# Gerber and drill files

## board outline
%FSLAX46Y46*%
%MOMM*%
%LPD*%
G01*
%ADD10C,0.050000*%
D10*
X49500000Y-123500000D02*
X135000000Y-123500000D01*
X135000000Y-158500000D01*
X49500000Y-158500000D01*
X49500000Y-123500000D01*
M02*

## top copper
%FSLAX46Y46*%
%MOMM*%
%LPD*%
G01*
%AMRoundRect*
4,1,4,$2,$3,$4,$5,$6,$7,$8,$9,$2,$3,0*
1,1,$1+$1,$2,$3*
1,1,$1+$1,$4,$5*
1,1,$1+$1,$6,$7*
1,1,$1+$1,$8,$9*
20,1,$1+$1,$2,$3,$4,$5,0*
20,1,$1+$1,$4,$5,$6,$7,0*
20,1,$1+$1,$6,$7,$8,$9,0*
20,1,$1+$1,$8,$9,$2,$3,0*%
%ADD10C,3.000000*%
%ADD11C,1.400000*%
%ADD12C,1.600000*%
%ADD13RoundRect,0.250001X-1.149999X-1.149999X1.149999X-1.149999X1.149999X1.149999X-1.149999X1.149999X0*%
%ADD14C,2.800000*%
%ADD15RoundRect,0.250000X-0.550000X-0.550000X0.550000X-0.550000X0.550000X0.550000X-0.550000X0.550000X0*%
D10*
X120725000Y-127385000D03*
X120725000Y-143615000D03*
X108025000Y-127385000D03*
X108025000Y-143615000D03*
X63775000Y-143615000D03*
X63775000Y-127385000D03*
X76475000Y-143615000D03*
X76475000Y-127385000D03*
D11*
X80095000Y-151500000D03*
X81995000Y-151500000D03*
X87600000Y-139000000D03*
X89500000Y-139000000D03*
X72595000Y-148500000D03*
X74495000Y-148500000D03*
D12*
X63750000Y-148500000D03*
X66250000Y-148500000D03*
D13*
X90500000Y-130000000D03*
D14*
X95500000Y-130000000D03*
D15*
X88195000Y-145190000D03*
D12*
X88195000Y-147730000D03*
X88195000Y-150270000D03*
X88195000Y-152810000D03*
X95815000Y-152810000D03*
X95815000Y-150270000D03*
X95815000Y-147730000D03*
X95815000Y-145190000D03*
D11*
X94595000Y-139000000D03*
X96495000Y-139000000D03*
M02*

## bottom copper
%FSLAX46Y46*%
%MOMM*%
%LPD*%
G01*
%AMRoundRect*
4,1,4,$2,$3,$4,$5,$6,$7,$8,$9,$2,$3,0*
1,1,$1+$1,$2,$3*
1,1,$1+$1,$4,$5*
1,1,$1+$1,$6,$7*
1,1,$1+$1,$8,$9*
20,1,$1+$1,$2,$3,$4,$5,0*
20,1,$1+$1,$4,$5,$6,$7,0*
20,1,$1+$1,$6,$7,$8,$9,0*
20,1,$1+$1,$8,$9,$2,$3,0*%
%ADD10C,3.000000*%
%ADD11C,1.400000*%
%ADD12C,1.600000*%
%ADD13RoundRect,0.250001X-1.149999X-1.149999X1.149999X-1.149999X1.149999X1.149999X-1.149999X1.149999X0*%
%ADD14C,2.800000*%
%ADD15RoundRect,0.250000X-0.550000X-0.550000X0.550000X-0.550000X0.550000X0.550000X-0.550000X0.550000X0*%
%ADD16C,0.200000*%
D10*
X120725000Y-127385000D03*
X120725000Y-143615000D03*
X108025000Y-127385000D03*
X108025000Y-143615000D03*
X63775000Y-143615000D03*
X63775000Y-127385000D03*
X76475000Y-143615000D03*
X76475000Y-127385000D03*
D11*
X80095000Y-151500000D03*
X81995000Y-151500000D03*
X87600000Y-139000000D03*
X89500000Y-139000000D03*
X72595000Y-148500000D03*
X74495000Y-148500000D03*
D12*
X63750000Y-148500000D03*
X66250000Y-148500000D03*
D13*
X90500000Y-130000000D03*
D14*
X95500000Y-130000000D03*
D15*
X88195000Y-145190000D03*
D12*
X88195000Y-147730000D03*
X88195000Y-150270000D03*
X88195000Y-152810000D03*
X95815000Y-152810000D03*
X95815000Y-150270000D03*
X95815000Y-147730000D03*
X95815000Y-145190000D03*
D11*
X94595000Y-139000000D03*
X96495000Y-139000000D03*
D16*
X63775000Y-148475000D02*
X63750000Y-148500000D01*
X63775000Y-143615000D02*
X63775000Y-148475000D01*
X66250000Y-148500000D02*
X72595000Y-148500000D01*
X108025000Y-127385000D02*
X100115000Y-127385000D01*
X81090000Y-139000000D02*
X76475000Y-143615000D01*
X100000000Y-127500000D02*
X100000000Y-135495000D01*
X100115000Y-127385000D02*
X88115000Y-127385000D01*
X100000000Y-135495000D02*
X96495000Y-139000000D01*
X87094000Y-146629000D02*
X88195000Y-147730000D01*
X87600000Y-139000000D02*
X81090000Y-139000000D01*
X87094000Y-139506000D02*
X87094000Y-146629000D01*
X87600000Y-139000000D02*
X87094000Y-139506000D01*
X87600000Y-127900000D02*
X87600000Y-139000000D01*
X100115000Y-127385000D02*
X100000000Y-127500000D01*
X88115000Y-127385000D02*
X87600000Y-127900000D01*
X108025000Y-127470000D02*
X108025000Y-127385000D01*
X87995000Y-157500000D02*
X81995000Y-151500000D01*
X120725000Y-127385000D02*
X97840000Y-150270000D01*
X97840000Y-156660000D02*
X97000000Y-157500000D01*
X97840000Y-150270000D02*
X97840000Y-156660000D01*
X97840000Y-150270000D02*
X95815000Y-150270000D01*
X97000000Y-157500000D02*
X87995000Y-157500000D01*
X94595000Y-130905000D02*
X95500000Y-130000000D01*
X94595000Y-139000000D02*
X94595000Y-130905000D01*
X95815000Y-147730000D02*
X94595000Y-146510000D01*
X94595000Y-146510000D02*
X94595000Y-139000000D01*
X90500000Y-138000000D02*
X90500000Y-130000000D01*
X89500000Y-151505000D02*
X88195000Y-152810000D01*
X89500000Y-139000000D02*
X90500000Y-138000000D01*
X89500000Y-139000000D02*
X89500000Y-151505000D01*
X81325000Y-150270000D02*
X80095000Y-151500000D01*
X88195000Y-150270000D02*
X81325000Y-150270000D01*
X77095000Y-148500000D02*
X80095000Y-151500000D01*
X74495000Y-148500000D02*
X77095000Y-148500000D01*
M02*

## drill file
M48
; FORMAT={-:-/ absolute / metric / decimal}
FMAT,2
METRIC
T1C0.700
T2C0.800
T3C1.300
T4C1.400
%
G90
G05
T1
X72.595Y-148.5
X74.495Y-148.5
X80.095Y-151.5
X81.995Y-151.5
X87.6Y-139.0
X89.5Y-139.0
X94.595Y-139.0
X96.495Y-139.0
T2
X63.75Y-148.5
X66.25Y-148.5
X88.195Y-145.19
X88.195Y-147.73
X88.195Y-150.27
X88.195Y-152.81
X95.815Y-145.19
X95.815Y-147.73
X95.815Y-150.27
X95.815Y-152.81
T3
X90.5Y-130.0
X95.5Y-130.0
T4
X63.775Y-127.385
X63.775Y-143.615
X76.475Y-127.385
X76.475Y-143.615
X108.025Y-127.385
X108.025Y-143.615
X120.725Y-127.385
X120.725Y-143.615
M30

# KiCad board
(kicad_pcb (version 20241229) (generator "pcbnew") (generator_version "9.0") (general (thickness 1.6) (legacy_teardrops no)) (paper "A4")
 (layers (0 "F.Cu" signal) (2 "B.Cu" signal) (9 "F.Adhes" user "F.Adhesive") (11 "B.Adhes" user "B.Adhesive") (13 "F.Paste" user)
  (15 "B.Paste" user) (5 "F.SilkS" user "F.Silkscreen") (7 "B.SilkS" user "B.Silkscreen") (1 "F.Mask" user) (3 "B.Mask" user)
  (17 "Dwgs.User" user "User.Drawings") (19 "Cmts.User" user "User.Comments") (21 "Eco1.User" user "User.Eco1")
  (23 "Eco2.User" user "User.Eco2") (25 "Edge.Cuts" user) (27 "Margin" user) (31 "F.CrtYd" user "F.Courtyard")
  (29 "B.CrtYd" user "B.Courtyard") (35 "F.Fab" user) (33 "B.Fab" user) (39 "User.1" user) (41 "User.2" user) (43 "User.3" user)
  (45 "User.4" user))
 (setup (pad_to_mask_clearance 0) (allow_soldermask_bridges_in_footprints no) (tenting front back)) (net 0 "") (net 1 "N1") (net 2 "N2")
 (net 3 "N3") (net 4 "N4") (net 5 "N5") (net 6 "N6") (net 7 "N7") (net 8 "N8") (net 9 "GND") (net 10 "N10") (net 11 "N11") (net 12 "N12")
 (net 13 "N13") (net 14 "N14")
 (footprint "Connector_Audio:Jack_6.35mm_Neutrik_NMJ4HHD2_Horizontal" (layer "F.Cu") (at 108.025 127.385)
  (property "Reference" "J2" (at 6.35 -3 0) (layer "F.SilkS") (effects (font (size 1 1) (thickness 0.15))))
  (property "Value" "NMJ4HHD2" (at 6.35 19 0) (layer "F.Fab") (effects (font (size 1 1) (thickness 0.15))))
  (pad "S" thru_hole circle (at 12.7 0) (size 3 3) (drill 1.4) (layers "*.Cu" "*.Mask") (remove_unused_layers no) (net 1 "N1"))
  (pad "SN" thru_hole circle (at 12.7 16.23) (size 3 3) (drill 1.4) (layers "*.Cu" "*.Mask") (remove_unused_layers no) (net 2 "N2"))
  (pad "T" thru_hole circle (at 0 0) (size 3 3) (drill 1.4) (layers "*.Cu" "*.Mask") (remove_unused_layers no) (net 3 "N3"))
  (pad "TN" thru_hole circle (at 0 16.23) (size 3 3) (drill 1.4) (layers "*.Cu" "*.Mask") (remove_unused_layers no) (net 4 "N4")))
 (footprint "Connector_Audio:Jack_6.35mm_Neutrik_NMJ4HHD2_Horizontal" (layer "F.Cu") (at 76.475 143.615 180)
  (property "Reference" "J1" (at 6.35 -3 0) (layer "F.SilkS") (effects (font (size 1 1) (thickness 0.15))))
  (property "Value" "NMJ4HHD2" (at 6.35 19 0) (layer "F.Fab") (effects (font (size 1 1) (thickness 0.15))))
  (pad "S" thru_hole circle (at 12.7 0 180) (size 3 3) (drill 1.4) (layers "*.Cu" "*.Mask") (remove_unused_layers no) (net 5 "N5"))
  (pad "SN" thru_hole circle (at 12.7 16.23 180) (size 3 3) (drill 1.4) (layers "*.Cu" "*.Mask") (remove_unused_layers no) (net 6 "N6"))
  (pad "T" thru_hole circle (at 0 0 180) (size 3 3) (drill 1.4) (layers "*.Cu" "*.Mask") (remove_unused_layers no) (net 3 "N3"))
  (pad "TN" thru_hole circle (at 0 16.23 180) (size 3 3) (drill 1.4) (layers "*.Cu" "*.Mask") (remove_unused_layers no) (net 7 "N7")))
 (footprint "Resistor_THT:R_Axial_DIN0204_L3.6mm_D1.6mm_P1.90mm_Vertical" (layer "F.Cu") (at 80.095 151.5)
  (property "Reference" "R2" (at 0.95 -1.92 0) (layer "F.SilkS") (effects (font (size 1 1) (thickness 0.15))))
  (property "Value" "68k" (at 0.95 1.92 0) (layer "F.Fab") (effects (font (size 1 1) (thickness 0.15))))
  (pad "1" thru_hole circle (at 0 0) (size 1.4 1.4) (drill 0.7) (layers "*.Cu" "*.Mask") (remove_unused_layers no) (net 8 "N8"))
  (pad "2" thru_hole circle (at 1.9 0) (size 1.4 1.4) (drill 0.7) (layers "*.Cu" "*.Mask") (remove_unused_layers no) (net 1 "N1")))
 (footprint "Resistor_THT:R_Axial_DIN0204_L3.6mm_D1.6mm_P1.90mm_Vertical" (layer "F.Cu") (at 87.6 139)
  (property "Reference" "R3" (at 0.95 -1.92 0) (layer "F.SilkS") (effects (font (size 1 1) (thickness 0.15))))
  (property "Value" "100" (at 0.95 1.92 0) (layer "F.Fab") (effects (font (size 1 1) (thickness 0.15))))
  (pad "1" thru_hole circle (at 0 0) (size 1.4 1.4) (drill 0.7) (layers "*.Cu" "*.Mask") (remove_unused_layers no) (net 3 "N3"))
  (pad "2" thru_hole circle (at 1.9 0) (size 1.4 1.4) (drill 0.7) (layers "*.Cu" "*.Mask") (remove_unused_layers no) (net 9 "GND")))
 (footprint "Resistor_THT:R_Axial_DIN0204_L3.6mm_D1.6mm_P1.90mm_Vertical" (layer "F.Cu") (at 72.595 148.5)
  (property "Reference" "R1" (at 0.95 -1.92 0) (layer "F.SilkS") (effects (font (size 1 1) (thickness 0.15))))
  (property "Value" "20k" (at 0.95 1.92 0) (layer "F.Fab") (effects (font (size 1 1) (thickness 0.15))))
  (pad "1" thru_hole circle (at 0 0) (size 1.4 1.4) (drill 0.7) (layers "*.Cu" "*.Mask") (remove_unused_layers no) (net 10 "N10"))
  (pad "2" thru_hole circle (at 1.9 0) (size 1.4 1.4) (drill 0.7) (layers "*.Cu" "*.Mask") (remove_unused_layers no) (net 8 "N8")))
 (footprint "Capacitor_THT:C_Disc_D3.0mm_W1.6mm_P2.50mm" (layer "F.Cu") (at 63.75 148.5)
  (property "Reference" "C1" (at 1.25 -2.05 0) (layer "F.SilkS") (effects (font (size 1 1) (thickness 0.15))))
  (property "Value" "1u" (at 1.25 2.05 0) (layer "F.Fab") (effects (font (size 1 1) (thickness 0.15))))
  (pad "1" thru_hole circle (at 0 0) (size 1.6 1.6) (drill 0.8) (layers "*.Cu" "*.Mask") (remove_unused_layers no) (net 5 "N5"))
  (pad "2" thru_hole circle (at 2.5 0) (size 1.6 1.6) (drill 0.8) (layers "*.Cu" "*.Mask") (remove_unused_layers no) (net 10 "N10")))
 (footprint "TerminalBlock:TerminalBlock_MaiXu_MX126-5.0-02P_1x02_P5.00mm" (layer "F.Cu") (at 90.5 130)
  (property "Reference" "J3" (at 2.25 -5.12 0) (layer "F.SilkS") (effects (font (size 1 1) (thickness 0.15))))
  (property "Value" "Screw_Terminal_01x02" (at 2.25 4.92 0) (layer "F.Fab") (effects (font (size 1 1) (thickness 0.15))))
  (pad "1" thru_hole roundrect (at 0 0) (size 2.8 2.8) (drill 1.3) (layers "*.Cu" "*.Mask") (remove_unused_layers no)
   (roundrect_rratio 0.089286) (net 9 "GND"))
  (pad "2" thru_hole circle (at 5 0) (size 2.8 2.8) (drill 1.3) (layers "*.Cu" "*.Mask") (remove_unused_layers no) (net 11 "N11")))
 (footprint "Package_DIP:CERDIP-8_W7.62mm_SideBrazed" (layer "F.Cu") (at 88.195 145.19)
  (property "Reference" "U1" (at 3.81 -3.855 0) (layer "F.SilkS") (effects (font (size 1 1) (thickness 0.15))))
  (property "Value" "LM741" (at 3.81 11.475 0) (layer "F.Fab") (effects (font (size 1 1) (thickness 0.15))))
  (pad "1" thru_hole roundrect (at 0 0) (size 1.6 1.6) (drill 0.8) (layers "*.Cu" "*.Mask") (remove_unused_layers no)
   (roundrect_rratio 0.15625) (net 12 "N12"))
  (pad "2" thru_hole circle (at 0 2.54) (size 1.6 1.6) (drill 0.8) (layers "*.Cu" "*.Mask") (remove_unused_layers no) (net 3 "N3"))
  (pad "3" thru_hole circle (at 0 5.08) (size 1.6 1.6) (drill 0.8) (layers "*.Cu" "*.Mask") (remove_unused_layers no) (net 8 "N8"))
  (pad "4" thru_hole circle (at 0 7.62) (size 1.6 1.6) (drill 0.8) (layers "*.Cu" "*.Mask") (remove_unused_layers no) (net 9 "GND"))
  (pad "5" thru_hole circle (at 7.62 7.62) (size 1.6 1.6) (drill 0.8) (layers "*.Cu" "*.Mask") (remove_unused_layers no) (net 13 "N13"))
  (pad "6" thru_hole circle (at 7.62 5.08) (size 1.6 1.6) (drill 0.8) (layers "*.Cu" "*.Mask") (remove_unused_layers no) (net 1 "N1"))
  (pad "7" thru_hole circle (at 7.62 2.54) (size 1.6 1.6) (drill 0.8) (layers "*.Cu" "*.Mask") (remove_unused_layers no) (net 11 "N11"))
  (pad "8" thru_hole circle (at 7.62 0) (size 1.6 1.6) (drill 0.8) (layers "*.Cu" "*.Mask") (remove_unused_layers no) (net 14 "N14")))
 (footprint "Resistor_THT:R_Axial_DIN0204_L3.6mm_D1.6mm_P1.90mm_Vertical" (layer "F.Cu") (at 94.595 139)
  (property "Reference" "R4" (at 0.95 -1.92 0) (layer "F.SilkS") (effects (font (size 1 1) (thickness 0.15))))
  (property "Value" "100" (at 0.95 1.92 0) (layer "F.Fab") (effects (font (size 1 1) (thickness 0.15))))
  (pad "1" thru_hole circle (at 0 0) (size 1.4 1.4) (drill 0.7) (layers "*.Cu" "*.Mask") (remove_unused_layers no) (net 11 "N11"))
  (pad "2" thru_hole circle (at 1.9 0) (size 1.4 1.4) (drill 0.7) (layers "*.Cu" "*.Mask") (remove_unused_layers no) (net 3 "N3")))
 (gr_rect (start 49.5 123.5) (end 135 158.5) (stroke (width 0.05) (type default)) (fill no) (layer "Edge.Cuts"))
 (segment (start 63.775 148.475) (end 63.75 148.5) (width 0.2) (layer "B.Cu") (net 5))
 (segment (start 63.775 143.615) (end 63.775 148.475) (width 0.2) (layer "B.Cu") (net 5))
 (segment (start 66.25 148.5) (end 72.595 148.5) (width 0.2) (layer "B.Cu") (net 10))
 (segment (start 108.025 127.385) (end 100.115 127.385) (width 0.2) (layer "B.Cu") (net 3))
 (segment (start 81.09 139) (end 76.475 143.615) (width 0.2) (layer "B.Cu") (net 3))
 (segment (start 100 127.5) (end 100 135.495) (width 0.2) (layer "B.Cu") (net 3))
 (segment (start 100.115 127.385) (end 88.115 127.385) (width 0.2) (layer "B.Cu") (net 3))
 (segment (start 100 135.495) (end 96.495 139) (width 0.2) (layer "B.Cu") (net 3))
 (segment (start 87.094 146.629) (end 88.195 147.73) (width 0.2) (layer "B.Cu") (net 3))
 (segment (start 87.6 139) (end 81.09 139) (width 0.2) (layer "B.Cu") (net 3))
 (segment (start 87.094 139.506) (end 87.094 146.629) (width 0.2) (layer "B.Cu") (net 3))
 (segment (start 87.6 139) (end 87.094 139.506) (width 0.2) (layer "B.Cu") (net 3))
 (segment (start 87.6 127.9) (end 87.6 139) (width 0.2) (layer "B.Cu") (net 3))
 (segment (start 100.115 127.385) (end 100 127.5) (width 0.2) (layer "B.Cu") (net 3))
 (segment (start 88.115 127.385) (end 87.6 127.9) (width 0.2) (layer "B.Cu") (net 3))
 (segment (start 108.025 127.47) (end 108.025 127.385) (width 0.2) (layer "B.Cu") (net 3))
 (segment (start 87.995 157.5) (end 81.995 151.5) (width 0.2) (layer "B.Cu") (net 1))
 (segment (start 120.725 127.385) (end 97.84 150.27) (width 0.2) (layer "B.Cu") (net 1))
 (segment (start 97.84 156.66) (end 97 157.5) (width 0.2) (layer "B.Cu") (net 1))
 (segment (start 97.84 150.27) (end 97.84 156.66) (width 0.2) (layer "B.Cu") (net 1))
 (segment (start 97.84 150.27) (end 95.815 150.27) (width 0.2) (layer "B.Cu") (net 1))
 (segment (start 97 157.5) (end 87.995 157.5) (width 0.2) (layer "B.Cu") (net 1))
 (segment (start 94.595 130.905) (end 95.5 130) (width 0.2) (layer "B.Cu") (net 11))
 (segment (start 94.595 139) (end 94.595 130.905) (width 0.2) (layer "B.Cu") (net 11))
 (segment (start 95.815 147.73) (end 94.595 146.51) (width 0.2) (layer "B.Cu") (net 11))
 (segment (start 94.595 146.51) (end 94.595 139) (width 0.2) (layer "B.Cu") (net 11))
 (segment (start 90.5 138) (end 90.5 130) (width 0.2) (layer "B.Cu") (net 9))
 (segment (start 89.5 151.505) (end 88.195 152.81) (width 0.2) (layer "B.Cu") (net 9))
 (segment (start 89.5 139) (end 90.5 138) (width 0.2) (layer "B.Cu") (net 9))
 (segment (start 89.5 139) (end 89.5 151.505) (width 0.2) (layer "B.Cu") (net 9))
 (segment (start 81.325 150.27) (end 80.095 151.5) (width 0.2) (layer "B.Cu") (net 8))
 (segment (start 88.195 150.27) (end 81.325 150.27) (width 0.2) (layer "B.Cu") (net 8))
 (segment (start 77.095 148.5) (end 80.095 151.5) (width 0.2) (layer "B.Cu") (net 8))
 (segment (start 74.495 148.5) (end 77.095 148.5) (width 0.2) (layer "B.Cu") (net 8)))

